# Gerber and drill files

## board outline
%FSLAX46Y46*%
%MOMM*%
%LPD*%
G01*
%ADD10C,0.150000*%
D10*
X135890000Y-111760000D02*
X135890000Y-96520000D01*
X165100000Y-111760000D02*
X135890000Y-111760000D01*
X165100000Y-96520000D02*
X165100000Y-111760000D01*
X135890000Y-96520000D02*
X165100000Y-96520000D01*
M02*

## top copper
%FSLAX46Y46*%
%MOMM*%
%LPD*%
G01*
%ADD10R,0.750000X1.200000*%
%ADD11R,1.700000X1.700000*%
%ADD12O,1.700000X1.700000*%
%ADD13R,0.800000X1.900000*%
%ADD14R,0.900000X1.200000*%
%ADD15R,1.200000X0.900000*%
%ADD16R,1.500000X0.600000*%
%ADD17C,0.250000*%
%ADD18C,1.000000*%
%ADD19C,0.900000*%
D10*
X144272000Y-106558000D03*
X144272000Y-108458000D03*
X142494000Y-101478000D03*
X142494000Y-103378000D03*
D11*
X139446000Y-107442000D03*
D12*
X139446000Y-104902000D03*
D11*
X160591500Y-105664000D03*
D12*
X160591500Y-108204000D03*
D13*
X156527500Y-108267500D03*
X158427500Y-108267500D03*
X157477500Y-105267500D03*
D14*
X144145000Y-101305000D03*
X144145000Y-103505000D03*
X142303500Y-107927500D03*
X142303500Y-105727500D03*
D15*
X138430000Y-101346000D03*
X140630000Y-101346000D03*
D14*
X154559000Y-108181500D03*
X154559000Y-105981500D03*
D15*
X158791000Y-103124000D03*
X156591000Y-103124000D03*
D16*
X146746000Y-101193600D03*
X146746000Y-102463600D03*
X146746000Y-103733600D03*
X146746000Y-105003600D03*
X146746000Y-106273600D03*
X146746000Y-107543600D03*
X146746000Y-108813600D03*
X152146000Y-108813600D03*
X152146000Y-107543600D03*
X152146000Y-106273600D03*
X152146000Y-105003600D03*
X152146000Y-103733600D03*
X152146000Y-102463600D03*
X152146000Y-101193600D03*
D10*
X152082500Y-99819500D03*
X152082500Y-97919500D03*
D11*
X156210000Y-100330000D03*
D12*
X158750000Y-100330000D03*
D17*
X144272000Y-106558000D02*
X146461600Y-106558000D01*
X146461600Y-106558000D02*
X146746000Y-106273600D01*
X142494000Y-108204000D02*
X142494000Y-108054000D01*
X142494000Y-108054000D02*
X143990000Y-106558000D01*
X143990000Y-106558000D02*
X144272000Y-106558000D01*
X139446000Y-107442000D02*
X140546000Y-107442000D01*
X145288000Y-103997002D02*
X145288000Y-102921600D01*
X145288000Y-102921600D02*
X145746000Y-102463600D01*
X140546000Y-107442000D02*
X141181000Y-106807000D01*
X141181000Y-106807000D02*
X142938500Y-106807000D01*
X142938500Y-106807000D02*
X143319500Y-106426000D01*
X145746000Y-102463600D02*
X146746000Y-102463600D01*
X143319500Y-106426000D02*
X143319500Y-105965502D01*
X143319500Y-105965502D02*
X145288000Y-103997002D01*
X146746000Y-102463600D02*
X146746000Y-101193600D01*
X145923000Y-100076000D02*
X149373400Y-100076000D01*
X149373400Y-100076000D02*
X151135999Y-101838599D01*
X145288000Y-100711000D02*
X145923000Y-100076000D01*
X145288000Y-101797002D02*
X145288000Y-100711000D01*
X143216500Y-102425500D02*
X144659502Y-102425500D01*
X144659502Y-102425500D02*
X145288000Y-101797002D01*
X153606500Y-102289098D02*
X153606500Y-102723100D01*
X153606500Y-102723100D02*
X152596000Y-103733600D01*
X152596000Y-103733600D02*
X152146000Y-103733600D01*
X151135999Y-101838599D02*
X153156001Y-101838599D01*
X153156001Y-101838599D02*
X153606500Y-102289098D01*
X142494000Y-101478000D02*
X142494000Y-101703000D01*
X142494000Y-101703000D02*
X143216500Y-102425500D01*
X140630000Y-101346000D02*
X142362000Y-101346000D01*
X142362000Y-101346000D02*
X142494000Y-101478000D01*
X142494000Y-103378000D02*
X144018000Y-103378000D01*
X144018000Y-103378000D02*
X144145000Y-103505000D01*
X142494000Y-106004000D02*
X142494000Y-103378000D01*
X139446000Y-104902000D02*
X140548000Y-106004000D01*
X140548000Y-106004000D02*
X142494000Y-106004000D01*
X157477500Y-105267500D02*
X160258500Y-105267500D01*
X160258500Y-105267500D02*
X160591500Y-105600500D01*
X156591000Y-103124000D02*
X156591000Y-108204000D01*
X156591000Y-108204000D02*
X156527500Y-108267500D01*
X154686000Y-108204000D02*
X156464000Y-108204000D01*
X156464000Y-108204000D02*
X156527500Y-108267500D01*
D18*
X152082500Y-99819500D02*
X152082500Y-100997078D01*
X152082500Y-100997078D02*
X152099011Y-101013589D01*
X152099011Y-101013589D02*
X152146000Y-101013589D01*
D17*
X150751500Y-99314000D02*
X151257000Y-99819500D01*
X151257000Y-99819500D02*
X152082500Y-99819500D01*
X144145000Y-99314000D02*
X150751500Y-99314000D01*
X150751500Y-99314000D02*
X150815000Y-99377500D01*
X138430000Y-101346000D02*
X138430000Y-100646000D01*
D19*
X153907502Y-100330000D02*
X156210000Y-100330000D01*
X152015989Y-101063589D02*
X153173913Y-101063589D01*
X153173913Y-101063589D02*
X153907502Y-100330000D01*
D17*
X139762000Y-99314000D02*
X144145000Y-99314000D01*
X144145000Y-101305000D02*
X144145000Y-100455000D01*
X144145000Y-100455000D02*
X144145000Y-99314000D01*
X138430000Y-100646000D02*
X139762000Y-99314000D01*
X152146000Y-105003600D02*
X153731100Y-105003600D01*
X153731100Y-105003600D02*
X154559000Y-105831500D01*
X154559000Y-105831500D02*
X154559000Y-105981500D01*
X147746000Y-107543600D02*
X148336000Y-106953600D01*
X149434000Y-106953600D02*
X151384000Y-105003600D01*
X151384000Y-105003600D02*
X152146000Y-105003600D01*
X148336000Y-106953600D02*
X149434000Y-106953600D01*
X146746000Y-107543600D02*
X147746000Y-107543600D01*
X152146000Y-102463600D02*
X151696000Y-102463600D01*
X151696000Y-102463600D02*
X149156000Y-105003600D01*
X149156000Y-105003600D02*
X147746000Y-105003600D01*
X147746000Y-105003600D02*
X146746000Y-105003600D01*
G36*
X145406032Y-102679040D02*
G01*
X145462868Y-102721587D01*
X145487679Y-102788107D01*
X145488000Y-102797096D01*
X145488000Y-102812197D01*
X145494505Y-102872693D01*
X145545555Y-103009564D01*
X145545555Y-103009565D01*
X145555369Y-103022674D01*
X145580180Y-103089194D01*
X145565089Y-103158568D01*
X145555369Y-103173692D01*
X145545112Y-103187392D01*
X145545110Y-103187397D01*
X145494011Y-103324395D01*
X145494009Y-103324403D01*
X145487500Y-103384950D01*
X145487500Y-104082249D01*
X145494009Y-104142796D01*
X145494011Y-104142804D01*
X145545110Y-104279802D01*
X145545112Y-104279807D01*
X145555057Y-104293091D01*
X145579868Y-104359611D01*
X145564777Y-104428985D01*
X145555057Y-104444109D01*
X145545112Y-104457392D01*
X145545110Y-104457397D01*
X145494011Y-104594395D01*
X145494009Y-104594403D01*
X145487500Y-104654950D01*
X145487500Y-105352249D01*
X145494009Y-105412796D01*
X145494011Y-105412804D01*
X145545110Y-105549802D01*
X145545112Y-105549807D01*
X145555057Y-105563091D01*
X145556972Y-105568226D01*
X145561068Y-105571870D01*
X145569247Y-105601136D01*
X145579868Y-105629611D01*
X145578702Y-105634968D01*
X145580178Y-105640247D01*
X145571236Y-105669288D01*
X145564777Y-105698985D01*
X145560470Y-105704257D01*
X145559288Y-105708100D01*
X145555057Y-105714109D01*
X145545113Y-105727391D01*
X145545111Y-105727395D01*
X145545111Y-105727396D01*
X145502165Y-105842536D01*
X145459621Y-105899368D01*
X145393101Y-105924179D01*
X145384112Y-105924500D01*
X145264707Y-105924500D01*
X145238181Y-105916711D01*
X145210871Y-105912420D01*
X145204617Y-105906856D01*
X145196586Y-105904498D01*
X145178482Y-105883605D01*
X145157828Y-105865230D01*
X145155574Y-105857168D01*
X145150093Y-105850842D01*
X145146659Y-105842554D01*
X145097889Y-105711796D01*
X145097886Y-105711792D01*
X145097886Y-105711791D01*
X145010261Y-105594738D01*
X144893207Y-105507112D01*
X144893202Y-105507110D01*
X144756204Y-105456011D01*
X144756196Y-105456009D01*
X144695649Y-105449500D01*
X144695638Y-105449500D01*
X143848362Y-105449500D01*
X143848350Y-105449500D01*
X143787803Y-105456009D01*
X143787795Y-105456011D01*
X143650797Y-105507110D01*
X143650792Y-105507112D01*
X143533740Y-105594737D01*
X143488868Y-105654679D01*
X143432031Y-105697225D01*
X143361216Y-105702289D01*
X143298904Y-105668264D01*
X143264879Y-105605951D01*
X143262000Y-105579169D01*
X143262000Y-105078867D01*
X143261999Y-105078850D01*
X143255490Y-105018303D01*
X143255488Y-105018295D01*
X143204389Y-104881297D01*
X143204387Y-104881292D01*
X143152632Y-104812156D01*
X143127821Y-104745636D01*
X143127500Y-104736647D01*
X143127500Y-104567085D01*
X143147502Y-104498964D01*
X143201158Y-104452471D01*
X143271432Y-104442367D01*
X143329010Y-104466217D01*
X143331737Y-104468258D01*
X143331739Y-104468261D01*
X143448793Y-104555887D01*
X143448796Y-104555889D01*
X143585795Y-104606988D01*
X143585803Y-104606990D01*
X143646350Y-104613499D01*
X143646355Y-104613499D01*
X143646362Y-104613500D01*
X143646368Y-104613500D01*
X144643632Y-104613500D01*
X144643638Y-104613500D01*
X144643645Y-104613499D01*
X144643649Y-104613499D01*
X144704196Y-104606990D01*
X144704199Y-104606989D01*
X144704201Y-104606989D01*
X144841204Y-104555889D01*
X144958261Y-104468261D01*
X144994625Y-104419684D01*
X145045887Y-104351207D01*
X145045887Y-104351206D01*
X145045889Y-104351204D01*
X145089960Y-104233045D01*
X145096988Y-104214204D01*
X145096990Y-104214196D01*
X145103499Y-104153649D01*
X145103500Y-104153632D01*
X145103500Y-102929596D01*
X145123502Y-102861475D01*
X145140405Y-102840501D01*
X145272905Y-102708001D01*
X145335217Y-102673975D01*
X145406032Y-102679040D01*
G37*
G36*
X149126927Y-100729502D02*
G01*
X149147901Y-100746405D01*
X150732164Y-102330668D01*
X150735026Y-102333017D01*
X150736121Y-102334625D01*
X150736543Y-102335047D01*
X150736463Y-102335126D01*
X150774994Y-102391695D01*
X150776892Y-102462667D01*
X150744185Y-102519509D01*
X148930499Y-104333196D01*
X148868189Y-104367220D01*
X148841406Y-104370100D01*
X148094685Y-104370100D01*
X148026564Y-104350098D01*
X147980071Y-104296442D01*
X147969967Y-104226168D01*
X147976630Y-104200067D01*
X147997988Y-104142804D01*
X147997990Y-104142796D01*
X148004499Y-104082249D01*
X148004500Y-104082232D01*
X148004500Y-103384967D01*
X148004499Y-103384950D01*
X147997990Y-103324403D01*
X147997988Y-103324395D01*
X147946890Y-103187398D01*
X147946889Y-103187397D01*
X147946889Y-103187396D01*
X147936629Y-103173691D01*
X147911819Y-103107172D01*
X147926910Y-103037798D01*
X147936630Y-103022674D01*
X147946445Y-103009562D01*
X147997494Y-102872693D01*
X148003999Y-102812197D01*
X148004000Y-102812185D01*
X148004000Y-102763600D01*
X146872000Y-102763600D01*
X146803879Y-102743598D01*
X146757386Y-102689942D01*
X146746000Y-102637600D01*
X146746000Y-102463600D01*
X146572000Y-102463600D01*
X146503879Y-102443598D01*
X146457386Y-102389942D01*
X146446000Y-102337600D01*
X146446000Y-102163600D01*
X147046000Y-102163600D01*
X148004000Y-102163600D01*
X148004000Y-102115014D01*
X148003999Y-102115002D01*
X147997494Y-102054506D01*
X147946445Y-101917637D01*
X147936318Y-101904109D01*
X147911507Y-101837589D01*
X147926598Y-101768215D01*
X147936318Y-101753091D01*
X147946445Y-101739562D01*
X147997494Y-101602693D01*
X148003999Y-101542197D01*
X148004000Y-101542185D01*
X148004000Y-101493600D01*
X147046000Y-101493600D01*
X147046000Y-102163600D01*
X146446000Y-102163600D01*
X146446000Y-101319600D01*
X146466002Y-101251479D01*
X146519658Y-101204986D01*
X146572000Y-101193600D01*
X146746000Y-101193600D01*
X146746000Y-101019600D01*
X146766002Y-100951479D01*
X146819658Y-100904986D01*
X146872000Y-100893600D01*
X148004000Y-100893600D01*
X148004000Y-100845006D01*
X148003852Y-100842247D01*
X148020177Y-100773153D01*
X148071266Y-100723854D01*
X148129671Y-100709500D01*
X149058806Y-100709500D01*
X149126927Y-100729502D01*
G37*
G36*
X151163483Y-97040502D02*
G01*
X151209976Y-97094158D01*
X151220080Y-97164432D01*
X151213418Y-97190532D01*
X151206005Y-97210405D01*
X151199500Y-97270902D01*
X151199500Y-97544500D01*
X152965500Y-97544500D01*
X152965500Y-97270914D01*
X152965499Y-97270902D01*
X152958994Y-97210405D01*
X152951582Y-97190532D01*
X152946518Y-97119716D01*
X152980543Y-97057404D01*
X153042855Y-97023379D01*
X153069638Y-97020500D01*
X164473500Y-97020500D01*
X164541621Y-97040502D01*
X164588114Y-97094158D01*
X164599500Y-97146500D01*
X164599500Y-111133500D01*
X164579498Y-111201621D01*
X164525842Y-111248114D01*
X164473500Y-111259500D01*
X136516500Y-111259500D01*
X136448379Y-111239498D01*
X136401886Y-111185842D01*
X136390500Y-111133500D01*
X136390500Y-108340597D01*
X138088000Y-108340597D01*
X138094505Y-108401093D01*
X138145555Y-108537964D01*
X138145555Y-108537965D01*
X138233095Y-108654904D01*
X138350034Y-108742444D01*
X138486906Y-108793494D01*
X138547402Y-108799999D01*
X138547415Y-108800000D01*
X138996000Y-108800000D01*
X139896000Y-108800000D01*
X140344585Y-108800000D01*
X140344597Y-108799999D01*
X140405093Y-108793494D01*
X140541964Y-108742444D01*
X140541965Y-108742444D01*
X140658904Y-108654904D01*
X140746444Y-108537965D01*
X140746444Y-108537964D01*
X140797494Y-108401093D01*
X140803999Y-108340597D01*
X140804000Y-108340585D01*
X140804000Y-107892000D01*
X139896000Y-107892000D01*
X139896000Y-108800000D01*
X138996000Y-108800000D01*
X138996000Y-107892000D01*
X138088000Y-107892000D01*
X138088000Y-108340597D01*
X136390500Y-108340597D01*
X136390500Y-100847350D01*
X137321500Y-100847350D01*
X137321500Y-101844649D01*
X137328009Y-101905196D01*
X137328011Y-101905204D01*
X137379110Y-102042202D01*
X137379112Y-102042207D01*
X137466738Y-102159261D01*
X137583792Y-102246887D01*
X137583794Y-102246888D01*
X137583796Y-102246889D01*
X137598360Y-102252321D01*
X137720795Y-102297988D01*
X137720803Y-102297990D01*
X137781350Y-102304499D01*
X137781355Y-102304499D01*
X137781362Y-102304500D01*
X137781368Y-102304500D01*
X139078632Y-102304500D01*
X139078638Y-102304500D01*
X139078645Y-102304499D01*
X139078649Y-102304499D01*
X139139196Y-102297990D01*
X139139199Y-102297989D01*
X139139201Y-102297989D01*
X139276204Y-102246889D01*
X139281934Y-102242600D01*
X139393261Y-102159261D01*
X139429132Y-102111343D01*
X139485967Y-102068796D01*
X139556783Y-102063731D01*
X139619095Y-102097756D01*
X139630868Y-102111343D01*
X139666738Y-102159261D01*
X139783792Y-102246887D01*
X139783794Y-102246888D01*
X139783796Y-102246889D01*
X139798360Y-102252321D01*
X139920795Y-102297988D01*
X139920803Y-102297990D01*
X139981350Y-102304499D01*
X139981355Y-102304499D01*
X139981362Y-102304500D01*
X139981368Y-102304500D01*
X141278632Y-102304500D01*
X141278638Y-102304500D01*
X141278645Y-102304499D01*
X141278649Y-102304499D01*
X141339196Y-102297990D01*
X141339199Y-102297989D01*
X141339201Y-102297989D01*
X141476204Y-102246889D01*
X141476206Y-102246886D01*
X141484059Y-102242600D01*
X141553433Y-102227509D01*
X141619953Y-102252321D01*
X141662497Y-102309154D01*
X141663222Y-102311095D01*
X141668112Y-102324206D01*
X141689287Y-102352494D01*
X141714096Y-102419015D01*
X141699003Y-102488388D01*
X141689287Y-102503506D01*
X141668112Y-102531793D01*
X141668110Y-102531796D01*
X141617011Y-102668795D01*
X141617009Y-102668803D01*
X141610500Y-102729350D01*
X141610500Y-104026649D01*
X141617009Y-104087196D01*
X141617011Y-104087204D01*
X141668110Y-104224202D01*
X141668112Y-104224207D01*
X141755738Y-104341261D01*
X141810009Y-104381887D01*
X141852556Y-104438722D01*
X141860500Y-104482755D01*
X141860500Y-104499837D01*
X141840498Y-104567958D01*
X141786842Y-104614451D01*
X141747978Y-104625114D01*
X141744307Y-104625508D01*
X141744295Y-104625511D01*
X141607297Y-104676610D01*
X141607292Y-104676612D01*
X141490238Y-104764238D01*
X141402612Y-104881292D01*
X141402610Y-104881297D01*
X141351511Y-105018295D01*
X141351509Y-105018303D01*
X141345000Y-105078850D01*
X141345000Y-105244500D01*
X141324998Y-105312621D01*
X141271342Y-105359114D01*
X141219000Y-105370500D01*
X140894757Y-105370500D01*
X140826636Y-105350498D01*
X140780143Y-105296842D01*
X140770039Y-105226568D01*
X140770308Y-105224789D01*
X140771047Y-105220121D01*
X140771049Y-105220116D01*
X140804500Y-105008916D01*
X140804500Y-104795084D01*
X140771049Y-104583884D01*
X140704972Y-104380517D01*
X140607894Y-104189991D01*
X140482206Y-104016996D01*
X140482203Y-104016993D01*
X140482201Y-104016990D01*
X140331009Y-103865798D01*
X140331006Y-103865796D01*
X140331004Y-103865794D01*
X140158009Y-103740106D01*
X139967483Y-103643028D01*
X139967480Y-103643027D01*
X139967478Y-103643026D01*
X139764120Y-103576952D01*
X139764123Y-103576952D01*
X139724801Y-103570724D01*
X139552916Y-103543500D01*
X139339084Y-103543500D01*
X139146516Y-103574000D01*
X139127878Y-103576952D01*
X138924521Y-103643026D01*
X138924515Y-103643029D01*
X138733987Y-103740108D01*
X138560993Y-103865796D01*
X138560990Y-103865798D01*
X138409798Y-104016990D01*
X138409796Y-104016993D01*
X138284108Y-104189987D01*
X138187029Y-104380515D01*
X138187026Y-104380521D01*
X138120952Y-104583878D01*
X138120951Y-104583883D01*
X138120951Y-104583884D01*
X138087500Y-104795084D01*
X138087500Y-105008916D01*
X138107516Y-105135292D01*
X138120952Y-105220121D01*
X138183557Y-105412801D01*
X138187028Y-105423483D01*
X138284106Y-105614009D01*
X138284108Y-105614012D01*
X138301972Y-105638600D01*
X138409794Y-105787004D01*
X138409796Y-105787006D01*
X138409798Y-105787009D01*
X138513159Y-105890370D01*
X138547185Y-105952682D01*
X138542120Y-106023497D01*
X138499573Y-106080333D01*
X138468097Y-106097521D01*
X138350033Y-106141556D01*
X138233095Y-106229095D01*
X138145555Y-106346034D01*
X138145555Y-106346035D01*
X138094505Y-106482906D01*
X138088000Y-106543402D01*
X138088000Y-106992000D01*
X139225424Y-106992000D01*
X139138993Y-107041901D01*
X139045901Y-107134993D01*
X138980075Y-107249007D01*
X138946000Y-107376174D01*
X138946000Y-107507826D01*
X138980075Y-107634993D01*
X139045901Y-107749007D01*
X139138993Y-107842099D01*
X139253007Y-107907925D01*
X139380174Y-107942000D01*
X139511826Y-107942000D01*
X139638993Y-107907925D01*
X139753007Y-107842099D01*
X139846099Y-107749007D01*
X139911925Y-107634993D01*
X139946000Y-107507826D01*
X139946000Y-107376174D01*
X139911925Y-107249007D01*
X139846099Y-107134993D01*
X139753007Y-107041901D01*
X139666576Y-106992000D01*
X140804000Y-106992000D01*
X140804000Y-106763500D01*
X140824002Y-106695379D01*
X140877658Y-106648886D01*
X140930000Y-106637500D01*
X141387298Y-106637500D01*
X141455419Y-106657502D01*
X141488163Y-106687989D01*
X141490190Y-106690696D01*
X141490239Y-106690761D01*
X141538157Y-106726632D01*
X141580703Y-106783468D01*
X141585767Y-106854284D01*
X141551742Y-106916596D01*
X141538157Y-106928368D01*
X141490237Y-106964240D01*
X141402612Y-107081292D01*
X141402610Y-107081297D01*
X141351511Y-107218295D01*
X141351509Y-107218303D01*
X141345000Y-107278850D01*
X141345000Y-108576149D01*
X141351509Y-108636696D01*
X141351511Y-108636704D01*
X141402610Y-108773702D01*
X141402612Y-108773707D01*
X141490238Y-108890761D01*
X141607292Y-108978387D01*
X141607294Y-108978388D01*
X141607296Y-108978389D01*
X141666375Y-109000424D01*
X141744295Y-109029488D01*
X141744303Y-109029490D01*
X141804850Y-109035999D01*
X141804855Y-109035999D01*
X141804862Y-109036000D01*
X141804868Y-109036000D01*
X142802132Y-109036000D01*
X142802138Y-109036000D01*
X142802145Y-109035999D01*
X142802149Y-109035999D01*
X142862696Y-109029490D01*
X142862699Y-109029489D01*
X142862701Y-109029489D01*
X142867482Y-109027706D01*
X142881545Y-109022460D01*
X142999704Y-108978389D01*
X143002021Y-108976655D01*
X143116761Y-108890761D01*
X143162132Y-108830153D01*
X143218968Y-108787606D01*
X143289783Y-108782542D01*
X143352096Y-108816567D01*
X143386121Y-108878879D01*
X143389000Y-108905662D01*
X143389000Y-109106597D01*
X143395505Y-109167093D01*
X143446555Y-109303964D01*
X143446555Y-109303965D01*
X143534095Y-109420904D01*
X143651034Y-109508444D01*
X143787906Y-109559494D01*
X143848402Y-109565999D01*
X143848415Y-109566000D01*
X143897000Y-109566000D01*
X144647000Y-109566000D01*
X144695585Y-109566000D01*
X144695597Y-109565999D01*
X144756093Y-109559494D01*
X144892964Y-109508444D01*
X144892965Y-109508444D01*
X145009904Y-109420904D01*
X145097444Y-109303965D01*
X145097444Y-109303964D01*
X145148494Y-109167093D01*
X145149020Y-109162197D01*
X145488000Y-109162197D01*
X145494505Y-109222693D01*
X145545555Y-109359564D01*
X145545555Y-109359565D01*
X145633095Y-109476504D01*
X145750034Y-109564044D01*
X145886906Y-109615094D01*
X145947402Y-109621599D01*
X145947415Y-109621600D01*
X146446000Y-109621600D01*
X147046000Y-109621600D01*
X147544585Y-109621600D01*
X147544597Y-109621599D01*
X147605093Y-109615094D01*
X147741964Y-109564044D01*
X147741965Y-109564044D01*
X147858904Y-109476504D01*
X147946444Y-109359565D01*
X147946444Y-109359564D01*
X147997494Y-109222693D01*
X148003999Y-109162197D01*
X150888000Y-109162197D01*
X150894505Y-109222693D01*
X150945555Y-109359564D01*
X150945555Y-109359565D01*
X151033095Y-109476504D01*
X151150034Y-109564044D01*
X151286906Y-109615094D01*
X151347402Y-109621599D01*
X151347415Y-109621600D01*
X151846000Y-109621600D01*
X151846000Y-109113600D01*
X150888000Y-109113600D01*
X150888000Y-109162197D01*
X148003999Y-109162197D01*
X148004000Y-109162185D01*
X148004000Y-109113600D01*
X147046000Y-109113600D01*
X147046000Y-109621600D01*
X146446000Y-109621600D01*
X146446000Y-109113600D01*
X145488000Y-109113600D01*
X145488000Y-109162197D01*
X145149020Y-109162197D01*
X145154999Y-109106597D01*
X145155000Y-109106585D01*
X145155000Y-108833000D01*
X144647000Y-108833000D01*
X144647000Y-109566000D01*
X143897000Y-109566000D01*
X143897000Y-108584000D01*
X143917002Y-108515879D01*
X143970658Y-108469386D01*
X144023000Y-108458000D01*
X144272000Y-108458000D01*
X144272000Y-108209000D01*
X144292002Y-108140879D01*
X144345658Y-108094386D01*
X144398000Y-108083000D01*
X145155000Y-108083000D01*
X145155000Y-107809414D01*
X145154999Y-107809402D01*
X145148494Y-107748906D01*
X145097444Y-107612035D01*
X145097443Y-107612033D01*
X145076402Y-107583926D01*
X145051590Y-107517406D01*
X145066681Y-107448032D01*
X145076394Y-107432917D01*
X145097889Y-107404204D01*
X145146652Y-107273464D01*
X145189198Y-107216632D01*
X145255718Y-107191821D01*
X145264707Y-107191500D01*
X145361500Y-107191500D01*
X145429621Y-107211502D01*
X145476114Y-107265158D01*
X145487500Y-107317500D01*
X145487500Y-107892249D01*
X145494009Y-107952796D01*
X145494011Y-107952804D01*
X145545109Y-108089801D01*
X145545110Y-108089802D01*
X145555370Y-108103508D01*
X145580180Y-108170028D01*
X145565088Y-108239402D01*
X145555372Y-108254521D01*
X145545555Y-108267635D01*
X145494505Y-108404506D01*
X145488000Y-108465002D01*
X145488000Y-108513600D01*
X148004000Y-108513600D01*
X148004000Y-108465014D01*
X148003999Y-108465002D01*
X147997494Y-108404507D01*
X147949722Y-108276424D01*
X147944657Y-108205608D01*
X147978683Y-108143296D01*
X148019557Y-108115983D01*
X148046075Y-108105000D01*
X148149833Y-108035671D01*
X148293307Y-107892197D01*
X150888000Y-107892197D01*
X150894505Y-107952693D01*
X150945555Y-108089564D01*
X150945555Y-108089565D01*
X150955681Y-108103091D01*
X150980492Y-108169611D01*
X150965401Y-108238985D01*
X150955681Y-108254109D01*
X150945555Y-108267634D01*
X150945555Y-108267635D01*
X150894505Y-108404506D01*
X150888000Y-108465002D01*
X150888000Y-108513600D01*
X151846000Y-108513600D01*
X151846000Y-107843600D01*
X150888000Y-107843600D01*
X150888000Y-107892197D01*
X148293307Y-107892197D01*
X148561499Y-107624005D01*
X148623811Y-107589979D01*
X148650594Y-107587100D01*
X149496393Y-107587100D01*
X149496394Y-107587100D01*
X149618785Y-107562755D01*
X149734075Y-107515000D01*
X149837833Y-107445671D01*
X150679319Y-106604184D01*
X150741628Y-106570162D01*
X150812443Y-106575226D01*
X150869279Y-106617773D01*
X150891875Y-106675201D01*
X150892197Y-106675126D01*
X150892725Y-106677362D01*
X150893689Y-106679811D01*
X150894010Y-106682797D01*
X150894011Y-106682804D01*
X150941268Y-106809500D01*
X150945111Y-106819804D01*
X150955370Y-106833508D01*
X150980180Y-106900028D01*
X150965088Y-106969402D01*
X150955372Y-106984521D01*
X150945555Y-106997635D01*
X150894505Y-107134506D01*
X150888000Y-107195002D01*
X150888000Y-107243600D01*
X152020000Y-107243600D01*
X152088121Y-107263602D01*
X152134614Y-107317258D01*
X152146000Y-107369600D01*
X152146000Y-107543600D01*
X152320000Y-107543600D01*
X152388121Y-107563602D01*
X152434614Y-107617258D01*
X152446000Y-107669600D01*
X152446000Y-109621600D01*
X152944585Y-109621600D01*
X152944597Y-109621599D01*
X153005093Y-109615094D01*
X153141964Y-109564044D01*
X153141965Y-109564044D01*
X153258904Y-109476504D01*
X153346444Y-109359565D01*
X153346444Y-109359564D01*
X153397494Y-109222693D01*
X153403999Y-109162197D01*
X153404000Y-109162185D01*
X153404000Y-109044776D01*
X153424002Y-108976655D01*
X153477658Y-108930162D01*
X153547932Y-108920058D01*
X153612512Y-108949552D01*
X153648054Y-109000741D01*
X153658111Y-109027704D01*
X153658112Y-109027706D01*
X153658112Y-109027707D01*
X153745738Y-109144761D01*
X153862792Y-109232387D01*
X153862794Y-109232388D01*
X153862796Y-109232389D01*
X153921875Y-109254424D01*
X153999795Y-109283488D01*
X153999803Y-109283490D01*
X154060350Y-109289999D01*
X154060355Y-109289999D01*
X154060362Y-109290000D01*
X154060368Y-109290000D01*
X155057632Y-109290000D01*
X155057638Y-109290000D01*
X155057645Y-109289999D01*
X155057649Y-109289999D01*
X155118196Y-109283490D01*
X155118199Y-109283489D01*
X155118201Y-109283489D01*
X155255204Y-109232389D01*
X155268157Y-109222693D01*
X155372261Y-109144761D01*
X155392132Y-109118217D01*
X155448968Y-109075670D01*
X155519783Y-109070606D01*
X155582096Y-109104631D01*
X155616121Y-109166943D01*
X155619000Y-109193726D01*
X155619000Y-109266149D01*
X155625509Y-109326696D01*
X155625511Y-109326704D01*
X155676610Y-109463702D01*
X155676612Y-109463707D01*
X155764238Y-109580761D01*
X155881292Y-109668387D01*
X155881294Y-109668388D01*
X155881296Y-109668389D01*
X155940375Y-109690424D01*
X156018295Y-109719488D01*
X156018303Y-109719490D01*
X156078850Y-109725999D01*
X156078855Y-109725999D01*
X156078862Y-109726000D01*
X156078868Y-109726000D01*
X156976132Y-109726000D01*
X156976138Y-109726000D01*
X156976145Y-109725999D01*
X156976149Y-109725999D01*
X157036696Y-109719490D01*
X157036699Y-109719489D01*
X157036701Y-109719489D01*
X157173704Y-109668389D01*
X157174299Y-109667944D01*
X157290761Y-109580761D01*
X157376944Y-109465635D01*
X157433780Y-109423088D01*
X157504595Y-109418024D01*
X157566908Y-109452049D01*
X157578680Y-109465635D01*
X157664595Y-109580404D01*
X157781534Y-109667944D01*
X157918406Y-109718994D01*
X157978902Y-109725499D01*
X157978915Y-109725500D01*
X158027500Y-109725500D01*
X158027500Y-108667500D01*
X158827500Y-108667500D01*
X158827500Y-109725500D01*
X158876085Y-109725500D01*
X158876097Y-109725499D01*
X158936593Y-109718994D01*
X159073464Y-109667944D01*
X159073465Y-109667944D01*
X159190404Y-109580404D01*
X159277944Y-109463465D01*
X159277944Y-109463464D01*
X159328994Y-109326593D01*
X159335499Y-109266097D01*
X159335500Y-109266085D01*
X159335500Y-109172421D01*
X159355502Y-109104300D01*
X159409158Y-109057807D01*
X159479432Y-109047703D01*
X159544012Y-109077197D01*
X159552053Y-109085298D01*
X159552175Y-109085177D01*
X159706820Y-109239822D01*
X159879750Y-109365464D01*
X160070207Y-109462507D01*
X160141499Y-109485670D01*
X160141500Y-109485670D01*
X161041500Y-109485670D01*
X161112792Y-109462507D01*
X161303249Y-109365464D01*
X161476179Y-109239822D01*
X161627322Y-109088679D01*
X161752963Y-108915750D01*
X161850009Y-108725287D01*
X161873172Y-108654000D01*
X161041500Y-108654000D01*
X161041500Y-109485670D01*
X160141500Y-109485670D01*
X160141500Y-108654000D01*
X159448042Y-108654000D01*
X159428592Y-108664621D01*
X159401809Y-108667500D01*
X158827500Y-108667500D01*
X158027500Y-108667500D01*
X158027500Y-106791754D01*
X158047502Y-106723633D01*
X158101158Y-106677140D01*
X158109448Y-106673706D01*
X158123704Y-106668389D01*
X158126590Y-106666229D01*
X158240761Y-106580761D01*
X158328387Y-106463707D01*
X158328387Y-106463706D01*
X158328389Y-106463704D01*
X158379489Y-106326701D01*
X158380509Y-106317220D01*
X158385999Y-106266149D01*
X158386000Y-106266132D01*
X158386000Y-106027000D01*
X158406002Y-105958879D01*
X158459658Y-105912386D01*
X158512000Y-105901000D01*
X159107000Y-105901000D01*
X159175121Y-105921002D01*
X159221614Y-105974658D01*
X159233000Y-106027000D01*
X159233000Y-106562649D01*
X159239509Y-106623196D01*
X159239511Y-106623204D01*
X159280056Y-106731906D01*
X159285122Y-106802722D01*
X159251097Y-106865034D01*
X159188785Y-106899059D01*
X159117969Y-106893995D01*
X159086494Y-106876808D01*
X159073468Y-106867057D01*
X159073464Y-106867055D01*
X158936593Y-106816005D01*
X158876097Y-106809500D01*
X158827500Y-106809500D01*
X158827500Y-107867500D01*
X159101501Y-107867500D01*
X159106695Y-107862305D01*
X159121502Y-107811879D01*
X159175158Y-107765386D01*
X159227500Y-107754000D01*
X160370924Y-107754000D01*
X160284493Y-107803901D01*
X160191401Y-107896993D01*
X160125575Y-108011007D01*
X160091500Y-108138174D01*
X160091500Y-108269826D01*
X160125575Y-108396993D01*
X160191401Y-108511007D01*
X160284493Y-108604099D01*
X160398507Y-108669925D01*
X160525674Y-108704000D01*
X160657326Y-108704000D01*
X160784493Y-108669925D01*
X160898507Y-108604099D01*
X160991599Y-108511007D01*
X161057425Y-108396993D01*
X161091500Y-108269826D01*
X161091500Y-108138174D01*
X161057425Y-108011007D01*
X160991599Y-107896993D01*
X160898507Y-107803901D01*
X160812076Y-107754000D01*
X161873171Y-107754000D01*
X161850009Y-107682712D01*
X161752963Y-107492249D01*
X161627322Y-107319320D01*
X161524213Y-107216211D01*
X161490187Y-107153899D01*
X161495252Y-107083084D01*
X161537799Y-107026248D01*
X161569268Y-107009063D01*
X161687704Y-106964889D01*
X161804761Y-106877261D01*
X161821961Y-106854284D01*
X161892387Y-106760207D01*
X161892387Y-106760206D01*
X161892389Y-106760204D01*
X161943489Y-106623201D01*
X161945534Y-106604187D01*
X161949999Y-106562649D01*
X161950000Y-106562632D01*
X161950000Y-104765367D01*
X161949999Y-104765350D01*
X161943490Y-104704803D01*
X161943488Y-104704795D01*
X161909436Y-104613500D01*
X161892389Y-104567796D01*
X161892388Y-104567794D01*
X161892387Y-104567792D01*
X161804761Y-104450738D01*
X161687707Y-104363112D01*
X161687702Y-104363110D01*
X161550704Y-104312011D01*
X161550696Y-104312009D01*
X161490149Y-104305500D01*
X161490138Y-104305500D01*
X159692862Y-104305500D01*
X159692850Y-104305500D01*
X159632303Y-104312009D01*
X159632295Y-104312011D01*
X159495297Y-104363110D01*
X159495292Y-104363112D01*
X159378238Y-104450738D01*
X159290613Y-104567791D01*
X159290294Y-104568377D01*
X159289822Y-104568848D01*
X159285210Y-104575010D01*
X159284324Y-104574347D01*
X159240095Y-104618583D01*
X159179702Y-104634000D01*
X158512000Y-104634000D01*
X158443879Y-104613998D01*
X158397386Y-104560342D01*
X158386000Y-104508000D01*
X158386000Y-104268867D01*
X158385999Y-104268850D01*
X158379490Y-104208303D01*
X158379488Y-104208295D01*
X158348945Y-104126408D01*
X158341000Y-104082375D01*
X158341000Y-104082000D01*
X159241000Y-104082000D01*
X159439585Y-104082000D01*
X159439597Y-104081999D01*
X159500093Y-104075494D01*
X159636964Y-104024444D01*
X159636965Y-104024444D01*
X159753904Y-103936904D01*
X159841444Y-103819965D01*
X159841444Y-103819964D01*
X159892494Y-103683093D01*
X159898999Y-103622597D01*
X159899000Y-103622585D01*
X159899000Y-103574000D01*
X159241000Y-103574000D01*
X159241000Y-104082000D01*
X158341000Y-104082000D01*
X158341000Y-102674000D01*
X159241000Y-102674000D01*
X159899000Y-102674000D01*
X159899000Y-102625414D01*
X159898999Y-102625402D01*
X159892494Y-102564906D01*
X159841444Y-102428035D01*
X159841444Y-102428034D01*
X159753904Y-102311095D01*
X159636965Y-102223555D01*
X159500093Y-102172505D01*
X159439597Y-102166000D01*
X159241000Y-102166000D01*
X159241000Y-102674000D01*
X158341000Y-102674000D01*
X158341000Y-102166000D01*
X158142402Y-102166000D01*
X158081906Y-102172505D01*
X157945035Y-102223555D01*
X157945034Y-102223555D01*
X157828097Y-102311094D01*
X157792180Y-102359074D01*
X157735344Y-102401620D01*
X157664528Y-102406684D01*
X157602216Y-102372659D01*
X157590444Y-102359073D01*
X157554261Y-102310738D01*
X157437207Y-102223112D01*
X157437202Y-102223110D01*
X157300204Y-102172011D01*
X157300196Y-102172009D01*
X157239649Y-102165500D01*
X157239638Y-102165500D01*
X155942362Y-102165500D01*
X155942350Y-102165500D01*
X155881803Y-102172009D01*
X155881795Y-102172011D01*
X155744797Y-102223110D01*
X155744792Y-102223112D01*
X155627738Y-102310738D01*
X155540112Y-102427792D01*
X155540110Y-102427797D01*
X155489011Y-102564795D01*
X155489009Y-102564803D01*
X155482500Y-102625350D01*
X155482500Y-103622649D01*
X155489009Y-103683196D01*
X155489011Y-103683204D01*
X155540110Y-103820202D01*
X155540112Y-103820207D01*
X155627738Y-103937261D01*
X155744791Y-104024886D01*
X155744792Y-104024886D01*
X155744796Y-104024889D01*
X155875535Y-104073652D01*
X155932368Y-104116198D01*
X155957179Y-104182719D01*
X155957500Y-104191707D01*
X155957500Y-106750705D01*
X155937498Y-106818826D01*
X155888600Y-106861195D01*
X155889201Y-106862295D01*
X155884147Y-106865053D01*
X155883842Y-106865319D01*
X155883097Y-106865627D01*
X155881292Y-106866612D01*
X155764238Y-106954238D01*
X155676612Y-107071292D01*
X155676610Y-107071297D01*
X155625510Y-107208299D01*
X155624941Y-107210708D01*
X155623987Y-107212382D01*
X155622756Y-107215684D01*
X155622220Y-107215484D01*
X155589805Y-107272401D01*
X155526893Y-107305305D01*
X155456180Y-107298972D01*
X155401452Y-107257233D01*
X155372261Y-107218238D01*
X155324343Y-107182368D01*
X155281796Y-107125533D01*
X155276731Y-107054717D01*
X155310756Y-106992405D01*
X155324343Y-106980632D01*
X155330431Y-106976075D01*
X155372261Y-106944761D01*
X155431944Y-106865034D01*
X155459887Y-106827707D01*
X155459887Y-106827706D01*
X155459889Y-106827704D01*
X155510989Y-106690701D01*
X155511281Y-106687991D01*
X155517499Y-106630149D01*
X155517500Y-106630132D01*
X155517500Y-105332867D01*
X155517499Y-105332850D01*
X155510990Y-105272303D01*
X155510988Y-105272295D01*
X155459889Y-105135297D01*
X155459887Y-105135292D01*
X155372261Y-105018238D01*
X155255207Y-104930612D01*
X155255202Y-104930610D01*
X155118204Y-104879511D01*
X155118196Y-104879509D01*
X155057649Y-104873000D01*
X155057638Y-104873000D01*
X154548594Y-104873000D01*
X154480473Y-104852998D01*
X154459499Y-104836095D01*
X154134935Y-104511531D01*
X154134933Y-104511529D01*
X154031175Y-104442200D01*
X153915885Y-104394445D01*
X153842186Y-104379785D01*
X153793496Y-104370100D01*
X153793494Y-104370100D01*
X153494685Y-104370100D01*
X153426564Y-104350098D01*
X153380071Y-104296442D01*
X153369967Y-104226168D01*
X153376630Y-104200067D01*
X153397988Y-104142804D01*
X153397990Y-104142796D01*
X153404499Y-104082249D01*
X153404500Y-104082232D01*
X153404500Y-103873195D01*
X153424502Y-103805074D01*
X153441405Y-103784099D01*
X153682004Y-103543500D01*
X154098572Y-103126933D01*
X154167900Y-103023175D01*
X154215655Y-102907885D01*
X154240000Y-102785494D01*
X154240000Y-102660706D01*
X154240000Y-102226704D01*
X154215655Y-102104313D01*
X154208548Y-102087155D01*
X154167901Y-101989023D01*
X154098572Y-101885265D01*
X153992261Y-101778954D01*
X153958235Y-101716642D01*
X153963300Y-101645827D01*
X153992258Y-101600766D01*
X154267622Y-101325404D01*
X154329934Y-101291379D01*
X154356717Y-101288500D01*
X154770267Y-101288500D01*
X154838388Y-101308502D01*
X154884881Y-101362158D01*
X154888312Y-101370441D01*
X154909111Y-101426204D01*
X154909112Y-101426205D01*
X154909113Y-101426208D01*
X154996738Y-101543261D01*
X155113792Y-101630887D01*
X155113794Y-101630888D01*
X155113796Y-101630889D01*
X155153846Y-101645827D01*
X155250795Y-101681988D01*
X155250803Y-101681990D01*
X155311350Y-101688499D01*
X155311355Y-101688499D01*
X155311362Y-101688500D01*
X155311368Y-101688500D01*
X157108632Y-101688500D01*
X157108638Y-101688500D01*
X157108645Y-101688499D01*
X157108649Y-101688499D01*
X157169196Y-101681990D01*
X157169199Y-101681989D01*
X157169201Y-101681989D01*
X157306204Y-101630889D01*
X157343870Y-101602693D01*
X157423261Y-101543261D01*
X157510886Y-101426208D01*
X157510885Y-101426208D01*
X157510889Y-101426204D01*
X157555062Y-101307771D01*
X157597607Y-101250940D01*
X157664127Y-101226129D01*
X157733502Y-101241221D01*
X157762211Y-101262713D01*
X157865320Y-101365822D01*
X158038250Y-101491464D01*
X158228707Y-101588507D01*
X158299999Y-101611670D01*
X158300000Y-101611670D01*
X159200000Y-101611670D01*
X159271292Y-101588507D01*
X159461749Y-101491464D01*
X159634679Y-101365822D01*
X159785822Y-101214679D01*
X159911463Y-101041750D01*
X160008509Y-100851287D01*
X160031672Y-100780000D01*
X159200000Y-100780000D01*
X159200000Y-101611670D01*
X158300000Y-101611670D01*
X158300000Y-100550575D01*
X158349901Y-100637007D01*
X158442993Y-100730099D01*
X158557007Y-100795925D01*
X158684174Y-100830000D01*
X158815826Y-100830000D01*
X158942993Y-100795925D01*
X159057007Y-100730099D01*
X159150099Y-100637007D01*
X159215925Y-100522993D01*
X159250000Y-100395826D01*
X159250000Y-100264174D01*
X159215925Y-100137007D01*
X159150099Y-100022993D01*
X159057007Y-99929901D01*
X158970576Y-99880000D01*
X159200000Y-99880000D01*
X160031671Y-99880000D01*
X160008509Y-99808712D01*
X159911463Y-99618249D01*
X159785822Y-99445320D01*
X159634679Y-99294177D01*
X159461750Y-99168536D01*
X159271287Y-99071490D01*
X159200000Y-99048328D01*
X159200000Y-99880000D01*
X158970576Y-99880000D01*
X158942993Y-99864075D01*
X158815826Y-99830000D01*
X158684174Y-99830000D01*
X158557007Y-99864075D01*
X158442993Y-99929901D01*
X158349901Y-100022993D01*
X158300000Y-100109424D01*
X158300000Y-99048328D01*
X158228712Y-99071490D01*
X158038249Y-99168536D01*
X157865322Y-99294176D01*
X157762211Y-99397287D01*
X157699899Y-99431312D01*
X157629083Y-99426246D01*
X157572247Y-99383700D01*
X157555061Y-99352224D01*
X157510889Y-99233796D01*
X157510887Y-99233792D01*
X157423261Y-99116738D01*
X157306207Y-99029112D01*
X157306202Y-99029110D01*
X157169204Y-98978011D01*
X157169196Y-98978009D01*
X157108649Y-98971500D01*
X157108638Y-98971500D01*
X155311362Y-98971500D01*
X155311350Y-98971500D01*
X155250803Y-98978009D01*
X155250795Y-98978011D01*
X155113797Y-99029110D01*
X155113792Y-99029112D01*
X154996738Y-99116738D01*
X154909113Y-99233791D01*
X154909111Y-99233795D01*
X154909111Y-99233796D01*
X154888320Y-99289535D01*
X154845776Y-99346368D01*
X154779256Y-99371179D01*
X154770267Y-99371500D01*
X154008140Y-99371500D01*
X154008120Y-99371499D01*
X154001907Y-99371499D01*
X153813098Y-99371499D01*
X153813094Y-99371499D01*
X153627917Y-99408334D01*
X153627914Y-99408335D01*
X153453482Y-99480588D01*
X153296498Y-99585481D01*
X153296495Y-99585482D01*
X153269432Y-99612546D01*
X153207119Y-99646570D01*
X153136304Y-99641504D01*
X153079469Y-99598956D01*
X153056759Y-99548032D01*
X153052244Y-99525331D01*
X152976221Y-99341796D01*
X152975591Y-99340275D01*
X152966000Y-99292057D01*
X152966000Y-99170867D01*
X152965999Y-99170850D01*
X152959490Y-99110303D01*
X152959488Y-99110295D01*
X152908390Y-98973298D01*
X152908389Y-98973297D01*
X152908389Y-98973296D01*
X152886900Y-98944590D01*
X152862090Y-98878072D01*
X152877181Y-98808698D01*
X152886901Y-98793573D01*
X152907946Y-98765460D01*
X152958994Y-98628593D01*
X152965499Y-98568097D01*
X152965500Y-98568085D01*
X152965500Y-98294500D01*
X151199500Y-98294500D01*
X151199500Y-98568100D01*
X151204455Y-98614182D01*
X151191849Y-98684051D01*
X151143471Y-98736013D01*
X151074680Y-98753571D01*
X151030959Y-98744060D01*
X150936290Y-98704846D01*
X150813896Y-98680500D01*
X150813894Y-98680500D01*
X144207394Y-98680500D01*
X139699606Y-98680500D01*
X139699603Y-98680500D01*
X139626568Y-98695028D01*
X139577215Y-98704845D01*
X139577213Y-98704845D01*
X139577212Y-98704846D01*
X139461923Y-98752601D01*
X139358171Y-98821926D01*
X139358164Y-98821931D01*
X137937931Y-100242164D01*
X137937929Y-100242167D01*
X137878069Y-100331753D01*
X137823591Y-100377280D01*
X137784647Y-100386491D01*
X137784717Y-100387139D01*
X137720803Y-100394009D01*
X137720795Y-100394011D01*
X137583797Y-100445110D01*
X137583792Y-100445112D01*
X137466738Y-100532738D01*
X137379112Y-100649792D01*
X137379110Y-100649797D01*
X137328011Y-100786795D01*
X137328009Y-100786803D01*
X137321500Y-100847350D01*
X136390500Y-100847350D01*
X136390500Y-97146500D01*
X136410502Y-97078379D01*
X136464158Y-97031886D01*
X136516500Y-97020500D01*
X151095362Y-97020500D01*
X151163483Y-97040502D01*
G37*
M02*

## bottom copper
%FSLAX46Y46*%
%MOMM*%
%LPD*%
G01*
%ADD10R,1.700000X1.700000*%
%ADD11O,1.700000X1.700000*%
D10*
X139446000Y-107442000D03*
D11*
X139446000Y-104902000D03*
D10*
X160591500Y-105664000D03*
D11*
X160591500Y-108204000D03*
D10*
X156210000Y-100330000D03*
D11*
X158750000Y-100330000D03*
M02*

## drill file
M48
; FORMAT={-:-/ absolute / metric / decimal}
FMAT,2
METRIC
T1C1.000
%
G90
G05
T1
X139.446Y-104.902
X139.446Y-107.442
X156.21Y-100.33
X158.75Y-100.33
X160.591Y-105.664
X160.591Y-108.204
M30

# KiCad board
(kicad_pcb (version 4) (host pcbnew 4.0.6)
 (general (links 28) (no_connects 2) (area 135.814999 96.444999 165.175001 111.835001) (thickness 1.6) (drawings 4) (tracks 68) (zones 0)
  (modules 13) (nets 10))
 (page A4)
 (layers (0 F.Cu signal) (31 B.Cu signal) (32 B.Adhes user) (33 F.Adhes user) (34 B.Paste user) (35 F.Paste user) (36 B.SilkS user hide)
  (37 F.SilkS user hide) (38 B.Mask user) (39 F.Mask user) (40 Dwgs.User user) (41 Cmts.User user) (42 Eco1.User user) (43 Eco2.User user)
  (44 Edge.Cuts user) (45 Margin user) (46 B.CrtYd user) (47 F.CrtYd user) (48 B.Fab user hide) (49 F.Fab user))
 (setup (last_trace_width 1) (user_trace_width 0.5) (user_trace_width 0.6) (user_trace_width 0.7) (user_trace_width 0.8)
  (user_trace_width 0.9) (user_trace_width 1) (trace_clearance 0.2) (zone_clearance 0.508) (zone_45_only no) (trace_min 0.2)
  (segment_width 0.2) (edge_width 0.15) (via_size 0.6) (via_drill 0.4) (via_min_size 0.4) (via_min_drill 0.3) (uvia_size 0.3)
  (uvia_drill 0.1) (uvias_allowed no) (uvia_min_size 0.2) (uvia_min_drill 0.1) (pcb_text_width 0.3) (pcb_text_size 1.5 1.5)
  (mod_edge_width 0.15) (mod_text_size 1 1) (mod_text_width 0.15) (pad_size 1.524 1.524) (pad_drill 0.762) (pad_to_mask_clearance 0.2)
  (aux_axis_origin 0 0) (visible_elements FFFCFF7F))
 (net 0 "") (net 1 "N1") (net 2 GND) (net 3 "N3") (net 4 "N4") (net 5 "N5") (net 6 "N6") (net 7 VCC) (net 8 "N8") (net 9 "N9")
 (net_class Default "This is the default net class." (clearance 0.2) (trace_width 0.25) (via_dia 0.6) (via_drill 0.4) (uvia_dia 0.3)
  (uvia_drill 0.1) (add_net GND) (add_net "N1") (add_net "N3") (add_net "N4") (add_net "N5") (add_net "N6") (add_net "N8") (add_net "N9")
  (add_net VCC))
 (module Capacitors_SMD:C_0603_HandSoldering (layer F.Cu) (at 144.272 107.508 270)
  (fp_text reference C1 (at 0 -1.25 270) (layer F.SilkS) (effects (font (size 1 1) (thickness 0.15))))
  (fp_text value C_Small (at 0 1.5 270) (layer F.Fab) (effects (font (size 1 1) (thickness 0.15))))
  (pad 1 smd rect (at -0.95 0 270) (size 1.2 0.75) (layers F.Cu F.Paste F.Mask) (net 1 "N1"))
  (pad 2 smd rect (at 0.95 0 270) (size 1.2 0.75) (layers F.Cu F.Paste F.Mask) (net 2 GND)))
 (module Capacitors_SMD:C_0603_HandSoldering (layer F.Cu) (at 142.494 102.428 270)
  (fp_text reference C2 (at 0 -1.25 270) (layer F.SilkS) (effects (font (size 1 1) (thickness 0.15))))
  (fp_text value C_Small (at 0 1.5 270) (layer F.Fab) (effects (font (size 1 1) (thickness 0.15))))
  (pad 1 smd rect (at -0.95 0 270) (size 1.2 0.75) (layers F.Cu F.Paste F.Mask) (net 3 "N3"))
  (pad 2 smd rect (at 0.95 0 270) (size 1.2 0.75) (layers F.Cu F.Paste F.Mask) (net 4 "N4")))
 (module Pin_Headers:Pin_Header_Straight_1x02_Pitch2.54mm (layer F.Cu) (at 139.446 107.442 180)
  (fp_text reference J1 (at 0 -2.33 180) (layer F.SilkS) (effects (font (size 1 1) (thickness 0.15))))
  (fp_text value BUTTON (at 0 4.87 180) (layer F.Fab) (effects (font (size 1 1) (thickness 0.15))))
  (pad 1 thru_hole rect (at 0 0 180) (size 1.7 1.7) (drill 1) (layers *.Cu *.Mask) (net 2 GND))
  (pad 2 thru_hole oval (at 0 2.54 180) (size 1.7 1.7) (drill 1) (layers *.Cu *.Mask) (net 4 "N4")))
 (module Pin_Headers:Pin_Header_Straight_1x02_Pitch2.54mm (layer F.Cu) (at 160.5915 105.664)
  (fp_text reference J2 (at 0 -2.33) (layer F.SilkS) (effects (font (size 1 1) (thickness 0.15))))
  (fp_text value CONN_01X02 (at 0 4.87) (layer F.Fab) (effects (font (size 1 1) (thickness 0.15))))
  (pad 1 thru_hole rect (at 0 0) (size 1.7 1.7) (drill 1) (layers *.Cu *.Mask) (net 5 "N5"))
  (pad 2 thru_hole oval (at 0 2.54) (size 1.7 1.7) (drill 1) (layers *.Cu *.Mask) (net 2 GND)))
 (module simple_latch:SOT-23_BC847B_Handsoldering (layer F.Cu) (at 157.4775 106.7675 90)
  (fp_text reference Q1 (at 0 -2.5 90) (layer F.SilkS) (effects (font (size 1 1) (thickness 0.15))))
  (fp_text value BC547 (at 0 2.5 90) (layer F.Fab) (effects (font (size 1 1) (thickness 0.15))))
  (pad 2 smd rect (at -1.5 -0.95 90) (size 1.9 0.8) (layers F.Cu F.Paste F.Mask) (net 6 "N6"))
  (pad 3 smd rect (at -1.5 0.95 90) (size 1.9 0.8) (layers F.Cu F.Paste F.Mask) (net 2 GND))
  (pad 1 smd rect (at 1.5 0 90) (size 1.9 0.8) (layers F.Cu F.Paste F.Mask) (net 5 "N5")))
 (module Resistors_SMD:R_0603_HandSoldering (layer F.Cu) (at 144.145 102.405 270)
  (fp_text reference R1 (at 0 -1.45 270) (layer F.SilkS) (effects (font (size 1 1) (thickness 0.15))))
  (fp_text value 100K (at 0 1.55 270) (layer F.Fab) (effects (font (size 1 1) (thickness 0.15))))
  (pad 1 smd rect (at -1.1 0 270) (size 1.2 0.9) (layers F.Cu F.Paste F.Mask) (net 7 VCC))
  (pad 2 smd rect (at 1.1 0 270) (size 1.2 0.9) (layers F.Cu F.Paste F.Mask) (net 4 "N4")))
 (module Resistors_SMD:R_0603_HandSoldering (layer F.Cu) (at 142.3035 106.8275 90)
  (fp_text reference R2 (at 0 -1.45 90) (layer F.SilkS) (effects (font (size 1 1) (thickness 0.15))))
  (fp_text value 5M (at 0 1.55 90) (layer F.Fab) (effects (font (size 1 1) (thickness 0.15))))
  (pad 1 smd rect (at -1.1 0 90) (size 1.2 0.9) (layers F.Cu F.Paste F.Mask) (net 1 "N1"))
  (pad 2 smd rect (at 1.1 0 90) (size 1.2 0.9) (layers F.Cu F.Paste F.Mask) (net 4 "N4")))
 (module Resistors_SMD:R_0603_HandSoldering (layer F.Cu) (at 139.53 101.346)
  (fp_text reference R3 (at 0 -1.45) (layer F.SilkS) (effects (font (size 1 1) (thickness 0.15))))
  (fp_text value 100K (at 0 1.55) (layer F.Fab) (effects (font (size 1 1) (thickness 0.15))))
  (pad 1 smd rect (at -1.1 0) (size 1.2 0.9) (layers F.Cu F.Paste F.Mask) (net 7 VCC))
  (pad 2 smd rect (at 1.1 0) (size 1.2 0.9) (layers F.Cu F.Paste F.Mask) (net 3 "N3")))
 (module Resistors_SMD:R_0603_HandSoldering (layer F.Cu) (at 154.559 107.0815 90)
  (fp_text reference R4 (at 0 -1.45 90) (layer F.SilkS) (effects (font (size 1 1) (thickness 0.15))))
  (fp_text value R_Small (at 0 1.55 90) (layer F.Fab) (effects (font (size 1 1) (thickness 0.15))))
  (pad 1 smd rect (at -1.1 0 90) (size 1.2 0.9) (layers F.Cu F.Paste F.Mask) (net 6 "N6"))
  (pad 2 smd rect (at 1.1 0 90) (size 1.2 0.9) (layers F.Cu F.Paste F.Mask) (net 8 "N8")))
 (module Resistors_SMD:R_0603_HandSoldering (layer F.Cu) (at 157.691 103.124 180)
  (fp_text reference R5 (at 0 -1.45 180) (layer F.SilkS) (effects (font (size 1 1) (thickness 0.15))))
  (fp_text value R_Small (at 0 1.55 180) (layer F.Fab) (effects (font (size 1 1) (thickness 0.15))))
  (pad 1 smd rect (at -1.1 0 180) (size 1.2 0.9) (layers F.Cu F.Paste F.Mask) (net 2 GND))
  (pad 2 smd rect (at 1.1 0 180) (size 1.2 0.9) (layers F.Cu F.Paste F.Mask) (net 6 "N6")))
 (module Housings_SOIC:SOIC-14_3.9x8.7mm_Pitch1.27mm (layer F.Cu) (at 149.446 105.0036)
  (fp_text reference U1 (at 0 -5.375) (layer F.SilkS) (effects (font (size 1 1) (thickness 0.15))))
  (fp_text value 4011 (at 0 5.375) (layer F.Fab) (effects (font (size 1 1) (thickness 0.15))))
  (pad 1 smd rect (at -2.7 -3.81) (size 1.5 0.6) (layers F.Cu F.Paste F.Mask) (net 2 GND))
  (pad 2 smd rect (at -2.7 -2.54) (size 1.5 0.6) (layers F.Cu F.Paste F.Mask) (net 2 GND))
  (pad 3 smd rect (at -2.7 -1.27) (size 1.5 0.6) (layers F.Cu F.Paste F.Mask))
  (pad 4 smd rect (at -2.7 0) (size 1.5 0.6) (layers F.Cu F.Paste F.Mask) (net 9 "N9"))
  (pad 5 smd rect (at -2.7 1.27) (size 1.5 0.6) (layers F.Cu F.Paste F.Mask) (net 1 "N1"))
  (pad 6 smd rect (at -2.7 2.54) (size 1.5 0.6) (layers F.Cu F.Paste F.Mask) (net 8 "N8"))
  (pad 7 smd rect (at -2.7 3.81) (size 1.5 0.6) (layers F.Cu F.Paste F.Mask) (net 2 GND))
  (pad 8 smd rect (at 2.7 3.81) (size 1.5 0.6) (layers F.Cu F.Paste F.Mask) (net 2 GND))
  (pad 9 smd rect (at 2.7 2.54) (size 1.5 0.6) (layers F.Cu F.Paste F.Mask) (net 2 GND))
  (pad 10 smd rect (at 2.7 1.27) (size 1.5 0.6) (layers F.Cu F.Paste F.Mask))
  (pad 11 smd rect (at 2.7 0) (size 1.5 0.6) (layers F.Cu F.Paste F.Mask) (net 8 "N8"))
  (pad 12 smd rect (at 2.7 -1.27) (size 1.5 0.6) (layers F.Cu F.Paste F.Mask) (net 3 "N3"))
  (pad 13 smd rect (at 2.7 -2.54) (size 1.5 0.6) (layers F.Cu F.Paste F.Mask) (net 9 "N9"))
  (pad 14 smd rect (at 2.7 -3.81) (size 1.5 0.6) (layers F.Cu F.Paste F.Mask) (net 7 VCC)))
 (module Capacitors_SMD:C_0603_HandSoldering (layer F.Cu) (at 152.0825 98.8695 90)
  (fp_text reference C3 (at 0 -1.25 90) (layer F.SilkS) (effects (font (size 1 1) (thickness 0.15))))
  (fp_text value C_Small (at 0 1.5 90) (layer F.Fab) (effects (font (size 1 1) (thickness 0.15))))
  (pad 1 smd rect (at -0.95 0 90) (size 1.2 0.75) (layers F.Cu F.Paste F.Mask) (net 7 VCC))
  (pad 2 smd rect (at 0.95 0 90) (size 1.2 0.75) (layers F.Cu F.Paste F.Mask) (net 2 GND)))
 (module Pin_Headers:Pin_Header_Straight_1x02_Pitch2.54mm (layer F.Cu) (at 156.21 100.33 90)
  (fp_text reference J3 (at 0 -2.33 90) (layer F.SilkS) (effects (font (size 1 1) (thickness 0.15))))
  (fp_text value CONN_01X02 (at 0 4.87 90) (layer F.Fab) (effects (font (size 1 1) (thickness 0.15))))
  (pad 1 thru_hole rect (at 0 0 90) (size 1.7 1.7) (drill 1) (layers *.Cu *.Mask) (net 7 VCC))
  (pad 2 thru_hole oval (at 0 2.54 90) (size 1.7 1.7) (drill 1) (layers *.Cu *.Mask) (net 2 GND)))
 (gr_line (start 135.89 111.76) (end 135.89 96.52) (layer Edge.Cuts) (width 0.15))
 (gr_line (start 165.1 111.76) (end 135.89 111.76) (layer Edge.Cuts) (width 0.15))
 (gr_line (start 165.1 96.52) (end 165.1 111.76) (layer Edge.Cuts) (width 0.15))
 (gr_line (start 135.89 96.52) (end 165.1 96.52) (layer Edge.Cuts) (width 0.15))
 (segment (start 144.272 106.558) (end 146.4616 106.558) (width 0.25) (layer F.Cu) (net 1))
 (segment (start 146.4616 106.558) (end 146.746 106.2736) (width 0.25) (layer F.Cu) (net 1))
 (segment (start 142.494 108.204) (end 142.494 108.054) (width 0.25) (layer F.Cu) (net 1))
 (segment (start 142.494 108.054) (end 143.99 106.558) (width 0.25) (layer F.Cu) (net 1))
 (segment (start 143.99 106.558) (end 144.272 106.558) (width 0.25) (layer F.Cu) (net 1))
 (segment (start 139.446 107.442) (end 140.546 107.442) (width 0.25) (layer F.Cu) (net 2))
 (segment (start 145.288 103.997002) (end 145.288 102.9216) (width 0.25) (layer F.Cu) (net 2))
 (segment (start 145.288 102.9216) (end 145.746 102.4636) (width 0.25) (layer F.Cu) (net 2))
 (segment (start 140.546 107.442) (end 141.181 106.807) (width 0.25) (layer F.Cu) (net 2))
 (segment (start 141.181 106.807) (end 142.9385 106.807) (width 0.25) (layer F.Cu) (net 2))
 (segment (start 142.9385 106.807) (end 143.3195 106.426) (width 0.25) (layer F.Cu) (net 2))
 (segment (start 145.746 102.4636) (end 146.746 102.4636) (width 0.25) (layer F.Cu) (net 2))
 (segment (start 143.3195 106.426) (end 143.3195 105.965502) (width 0.25) (layer F.Cu) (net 2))
 (segment (start 143.3195 105.965502) (end 145.288 103.997002) (width 0.25) (layer F.Cu) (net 2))
 (segment (start 146.746 102.4636) (end 146.746 101.1936) (width 0.25) (layer F.Cu) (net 2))
 (segment (start 145.923 100.076) (end 149.3734 100.076) (width 0.25) (layer F.Cu) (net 3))
 (segment (start 149.3734 100.076) (end 151.135999 101.838599) (width 0.25) (layer F.Cu) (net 3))
 (segment (start 145.288 100.711) (end 145.923 100.076) (width 0.25) (layer F.Cu) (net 3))
 (segment (start 145.288 101.797002) (end 145.288 100.711) (width 0.25) (layer F.Cu) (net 3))
 (segment (start 143.2165 102.4255) (end 144.659502 102.4255) (width 0.25) (layer F.Cu) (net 3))
 (segment (start 144.659502 102.4255) (end 145.288 101.797002) (width 0.25) (layer F.Cu) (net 3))
 (segment (start 153.6065 102.289098) (end 153.6065 102.7231) (width 0.25) (layer F.Cu) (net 3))
 (segment (start 153.6065 102.7231) (end 152.596 103.7336) (width 0.25) (layer F.Cu) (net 3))
 (segment (start 152.596 103.7336) (end 152.146 103.7336) (width 0.25) (layer F.Cu) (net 3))
 (segment (start 151.135999 101.838599) (end 153.156001 101.838599) (width 0.25) (layer F.Cu) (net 3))
 (segment (start 153.156001 101.838599) (end 153.6065 102.289098) (width 0.25) (layer F.Cu) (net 3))
 (segment (start 142.494 101.478) (end 142.494 101.703) (width 0.25) (layer F.Cu) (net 3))
 (segment (start 142.494 101.703) (end 143.2165 102.4255) (width 0.25) (layer F.Cu) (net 3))
 (segment (start 140.63 101.346) (end 142.362 101.346) (width 0.25) (layer F.Cu) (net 3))
 (segment (start 142.362 101.346) (end 142.494 101.478) (width 0.25) (layer F.Cu) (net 3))
 (segment (start 142.494 103.378) (end 144.018 103.378) (width 0.25) (layer F.Cu) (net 4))
 (segment (start 144.018 103.378) (end 144.145 103.505) (width 0.25) (layer F.Cu) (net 4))
 (segment (start 142.494 106.004) (end 142.494 103.378) (width 0.25) (layer F.Cu) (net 4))
 (segment (start 139.446 104.902) (end 140.548 106.004) (width 0.25) (layer F.Cu) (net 4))
 (segment (start 140.548 106.004) (end 142.494 106.004) (width 0.25) (layer F.Cu) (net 4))
 (segment (start 157.4775 105.2675) (end 160.2585 105.2675) (width 0.25) (layer F.Cu) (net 5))
 (segment (start 160.2585 105.2675) (end 160.5915 105.6005) (width 0.25) (layer F.Cu) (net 5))
 (segment (start 156.591 103.124) (end 156.591 108.204) (width 0.25) (layer F.Cu) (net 6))
 (segment (start 156.591 108.204) (end 156.5275 108.2675) (width 0.25) (layer F.Cu) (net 6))
 (segment (start 154.686 108.204) (end 156.464 108.204) (width 0.25) (layer F.Cu) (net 6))
 (segment (start 156.464 108.204) (end 156.5275 108.2675) (width 0.25) (layer F.Cu) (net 6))
 (segment (start 152.0825 99.8195) (end 152.0825 100.997078) (width 1) (layer F.Cu) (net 7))
 (segment (start 152.0825 100.997078) (end 152.099011 101.013589) (width 1) (layer F.Cu) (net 7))
 (segment (start 152.099011 101.013589) (end 152.146 101.013589) (width 1) (layer F.Cu) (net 7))
 (segment (start 150.7515 99.314) (end 151.257 99.8195) (width 0.25) (layer F.Cu) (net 7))
 (segment (start 151.257 99.8195) (end 152.0825 99.8195) (width 0.25) (layer F.Cu) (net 7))
 (segment (start 144.145 99.314) (end 150.7515 99.314) (width 0.25) (layer F.Cu) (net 7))
 (segment (start 150.7515 99.314) (end 150.815 99.3775) (width 0.25) (layer F.Cu) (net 7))
 (segment (start 138.43 101.346) (end 138.43 100.646) (width 0.25) (layer F.Cu) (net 7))
 (segment (start 153.907502 100.33) (end 156.21 100.33) (width 0.9) (layer F.Cu) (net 7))
 (segment (start 152.015989 101.063589) (end 153.173913 101.063589) (width 0.9) (layer F.Cu) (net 7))
 (segment (start 153.173913 101.063589) (end 153.907502 100.33) (width 0.9) (layer F.Cu) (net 7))
 (segment (start 139.762 99.314) (end 144.145 99.314) (width 0.25) (layer F.Cu) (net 7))
 (segment (start 144.145 101.305) (end 144.145 100.455) (width 0.25) (layer F.Cu) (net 7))
 (segment (start 144.145 100.455) (end 144.145 99.314) (width 0.25) (layer F.Cu) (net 7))
 (segment (start 138.43 100.646) (end 139.762 99.314) (width 0.25) (layer F.Cu) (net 7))
 (segment (start 152.146 105.0036) (end 153.7311 105.0036) (width 0.25) (layer F.Cu) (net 8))
 (segment (start 153.7311 105.0036) (end 154.559 105.8315) (width 0.25) (layer F.Cu) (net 8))
 (segment (start 154.559 105.8315) (end 154.559 105.9815) (width 0.25) (layer F.Cu) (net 8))
 (segment (start 147.746 107.5436) (end 148.336 106.9536) (width 0.25) (layer F.Cu) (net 8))
 (segment (start 149.434 106.9536) (end 151.384 105.0036) (width 0.25) (layer F.Cu) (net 8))
 (segment (start 151.384 105.0036) (end 152.146 105.0036) (width 0.25) (layer F.Cu) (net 8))
 (segment (start 148.336 106.9536) (end 149.434 106.9536) (width 0.25) (layer F.Cu) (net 8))
 (segment (start 146.746 107.5436) (end 147.746 107.5436) (width 0.25) (layer F.Cu) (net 8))
 (segment (start 152.146 102.4636) (end 151.696 102.4636) (width 0.25) (layer F.Cu) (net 9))
 (segment (start 151.696 102.4636) (end 149.156 105.0036) (width 0.25) (layer F.Cu) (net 9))
 (segment (start 149.156 105.0036) (end 147.746 105.0036) (width 0.25) (layer F.Cu) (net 9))
 (segment (start 147.746 105.0036) (end 146.746 105.0036) (width 0.25) (layer F.Cu) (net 9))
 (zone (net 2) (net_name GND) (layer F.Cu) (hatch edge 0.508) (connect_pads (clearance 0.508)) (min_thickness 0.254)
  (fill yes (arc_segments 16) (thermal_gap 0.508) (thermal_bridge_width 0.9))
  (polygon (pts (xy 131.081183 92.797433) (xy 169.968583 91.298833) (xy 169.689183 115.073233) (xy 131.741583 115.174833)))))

